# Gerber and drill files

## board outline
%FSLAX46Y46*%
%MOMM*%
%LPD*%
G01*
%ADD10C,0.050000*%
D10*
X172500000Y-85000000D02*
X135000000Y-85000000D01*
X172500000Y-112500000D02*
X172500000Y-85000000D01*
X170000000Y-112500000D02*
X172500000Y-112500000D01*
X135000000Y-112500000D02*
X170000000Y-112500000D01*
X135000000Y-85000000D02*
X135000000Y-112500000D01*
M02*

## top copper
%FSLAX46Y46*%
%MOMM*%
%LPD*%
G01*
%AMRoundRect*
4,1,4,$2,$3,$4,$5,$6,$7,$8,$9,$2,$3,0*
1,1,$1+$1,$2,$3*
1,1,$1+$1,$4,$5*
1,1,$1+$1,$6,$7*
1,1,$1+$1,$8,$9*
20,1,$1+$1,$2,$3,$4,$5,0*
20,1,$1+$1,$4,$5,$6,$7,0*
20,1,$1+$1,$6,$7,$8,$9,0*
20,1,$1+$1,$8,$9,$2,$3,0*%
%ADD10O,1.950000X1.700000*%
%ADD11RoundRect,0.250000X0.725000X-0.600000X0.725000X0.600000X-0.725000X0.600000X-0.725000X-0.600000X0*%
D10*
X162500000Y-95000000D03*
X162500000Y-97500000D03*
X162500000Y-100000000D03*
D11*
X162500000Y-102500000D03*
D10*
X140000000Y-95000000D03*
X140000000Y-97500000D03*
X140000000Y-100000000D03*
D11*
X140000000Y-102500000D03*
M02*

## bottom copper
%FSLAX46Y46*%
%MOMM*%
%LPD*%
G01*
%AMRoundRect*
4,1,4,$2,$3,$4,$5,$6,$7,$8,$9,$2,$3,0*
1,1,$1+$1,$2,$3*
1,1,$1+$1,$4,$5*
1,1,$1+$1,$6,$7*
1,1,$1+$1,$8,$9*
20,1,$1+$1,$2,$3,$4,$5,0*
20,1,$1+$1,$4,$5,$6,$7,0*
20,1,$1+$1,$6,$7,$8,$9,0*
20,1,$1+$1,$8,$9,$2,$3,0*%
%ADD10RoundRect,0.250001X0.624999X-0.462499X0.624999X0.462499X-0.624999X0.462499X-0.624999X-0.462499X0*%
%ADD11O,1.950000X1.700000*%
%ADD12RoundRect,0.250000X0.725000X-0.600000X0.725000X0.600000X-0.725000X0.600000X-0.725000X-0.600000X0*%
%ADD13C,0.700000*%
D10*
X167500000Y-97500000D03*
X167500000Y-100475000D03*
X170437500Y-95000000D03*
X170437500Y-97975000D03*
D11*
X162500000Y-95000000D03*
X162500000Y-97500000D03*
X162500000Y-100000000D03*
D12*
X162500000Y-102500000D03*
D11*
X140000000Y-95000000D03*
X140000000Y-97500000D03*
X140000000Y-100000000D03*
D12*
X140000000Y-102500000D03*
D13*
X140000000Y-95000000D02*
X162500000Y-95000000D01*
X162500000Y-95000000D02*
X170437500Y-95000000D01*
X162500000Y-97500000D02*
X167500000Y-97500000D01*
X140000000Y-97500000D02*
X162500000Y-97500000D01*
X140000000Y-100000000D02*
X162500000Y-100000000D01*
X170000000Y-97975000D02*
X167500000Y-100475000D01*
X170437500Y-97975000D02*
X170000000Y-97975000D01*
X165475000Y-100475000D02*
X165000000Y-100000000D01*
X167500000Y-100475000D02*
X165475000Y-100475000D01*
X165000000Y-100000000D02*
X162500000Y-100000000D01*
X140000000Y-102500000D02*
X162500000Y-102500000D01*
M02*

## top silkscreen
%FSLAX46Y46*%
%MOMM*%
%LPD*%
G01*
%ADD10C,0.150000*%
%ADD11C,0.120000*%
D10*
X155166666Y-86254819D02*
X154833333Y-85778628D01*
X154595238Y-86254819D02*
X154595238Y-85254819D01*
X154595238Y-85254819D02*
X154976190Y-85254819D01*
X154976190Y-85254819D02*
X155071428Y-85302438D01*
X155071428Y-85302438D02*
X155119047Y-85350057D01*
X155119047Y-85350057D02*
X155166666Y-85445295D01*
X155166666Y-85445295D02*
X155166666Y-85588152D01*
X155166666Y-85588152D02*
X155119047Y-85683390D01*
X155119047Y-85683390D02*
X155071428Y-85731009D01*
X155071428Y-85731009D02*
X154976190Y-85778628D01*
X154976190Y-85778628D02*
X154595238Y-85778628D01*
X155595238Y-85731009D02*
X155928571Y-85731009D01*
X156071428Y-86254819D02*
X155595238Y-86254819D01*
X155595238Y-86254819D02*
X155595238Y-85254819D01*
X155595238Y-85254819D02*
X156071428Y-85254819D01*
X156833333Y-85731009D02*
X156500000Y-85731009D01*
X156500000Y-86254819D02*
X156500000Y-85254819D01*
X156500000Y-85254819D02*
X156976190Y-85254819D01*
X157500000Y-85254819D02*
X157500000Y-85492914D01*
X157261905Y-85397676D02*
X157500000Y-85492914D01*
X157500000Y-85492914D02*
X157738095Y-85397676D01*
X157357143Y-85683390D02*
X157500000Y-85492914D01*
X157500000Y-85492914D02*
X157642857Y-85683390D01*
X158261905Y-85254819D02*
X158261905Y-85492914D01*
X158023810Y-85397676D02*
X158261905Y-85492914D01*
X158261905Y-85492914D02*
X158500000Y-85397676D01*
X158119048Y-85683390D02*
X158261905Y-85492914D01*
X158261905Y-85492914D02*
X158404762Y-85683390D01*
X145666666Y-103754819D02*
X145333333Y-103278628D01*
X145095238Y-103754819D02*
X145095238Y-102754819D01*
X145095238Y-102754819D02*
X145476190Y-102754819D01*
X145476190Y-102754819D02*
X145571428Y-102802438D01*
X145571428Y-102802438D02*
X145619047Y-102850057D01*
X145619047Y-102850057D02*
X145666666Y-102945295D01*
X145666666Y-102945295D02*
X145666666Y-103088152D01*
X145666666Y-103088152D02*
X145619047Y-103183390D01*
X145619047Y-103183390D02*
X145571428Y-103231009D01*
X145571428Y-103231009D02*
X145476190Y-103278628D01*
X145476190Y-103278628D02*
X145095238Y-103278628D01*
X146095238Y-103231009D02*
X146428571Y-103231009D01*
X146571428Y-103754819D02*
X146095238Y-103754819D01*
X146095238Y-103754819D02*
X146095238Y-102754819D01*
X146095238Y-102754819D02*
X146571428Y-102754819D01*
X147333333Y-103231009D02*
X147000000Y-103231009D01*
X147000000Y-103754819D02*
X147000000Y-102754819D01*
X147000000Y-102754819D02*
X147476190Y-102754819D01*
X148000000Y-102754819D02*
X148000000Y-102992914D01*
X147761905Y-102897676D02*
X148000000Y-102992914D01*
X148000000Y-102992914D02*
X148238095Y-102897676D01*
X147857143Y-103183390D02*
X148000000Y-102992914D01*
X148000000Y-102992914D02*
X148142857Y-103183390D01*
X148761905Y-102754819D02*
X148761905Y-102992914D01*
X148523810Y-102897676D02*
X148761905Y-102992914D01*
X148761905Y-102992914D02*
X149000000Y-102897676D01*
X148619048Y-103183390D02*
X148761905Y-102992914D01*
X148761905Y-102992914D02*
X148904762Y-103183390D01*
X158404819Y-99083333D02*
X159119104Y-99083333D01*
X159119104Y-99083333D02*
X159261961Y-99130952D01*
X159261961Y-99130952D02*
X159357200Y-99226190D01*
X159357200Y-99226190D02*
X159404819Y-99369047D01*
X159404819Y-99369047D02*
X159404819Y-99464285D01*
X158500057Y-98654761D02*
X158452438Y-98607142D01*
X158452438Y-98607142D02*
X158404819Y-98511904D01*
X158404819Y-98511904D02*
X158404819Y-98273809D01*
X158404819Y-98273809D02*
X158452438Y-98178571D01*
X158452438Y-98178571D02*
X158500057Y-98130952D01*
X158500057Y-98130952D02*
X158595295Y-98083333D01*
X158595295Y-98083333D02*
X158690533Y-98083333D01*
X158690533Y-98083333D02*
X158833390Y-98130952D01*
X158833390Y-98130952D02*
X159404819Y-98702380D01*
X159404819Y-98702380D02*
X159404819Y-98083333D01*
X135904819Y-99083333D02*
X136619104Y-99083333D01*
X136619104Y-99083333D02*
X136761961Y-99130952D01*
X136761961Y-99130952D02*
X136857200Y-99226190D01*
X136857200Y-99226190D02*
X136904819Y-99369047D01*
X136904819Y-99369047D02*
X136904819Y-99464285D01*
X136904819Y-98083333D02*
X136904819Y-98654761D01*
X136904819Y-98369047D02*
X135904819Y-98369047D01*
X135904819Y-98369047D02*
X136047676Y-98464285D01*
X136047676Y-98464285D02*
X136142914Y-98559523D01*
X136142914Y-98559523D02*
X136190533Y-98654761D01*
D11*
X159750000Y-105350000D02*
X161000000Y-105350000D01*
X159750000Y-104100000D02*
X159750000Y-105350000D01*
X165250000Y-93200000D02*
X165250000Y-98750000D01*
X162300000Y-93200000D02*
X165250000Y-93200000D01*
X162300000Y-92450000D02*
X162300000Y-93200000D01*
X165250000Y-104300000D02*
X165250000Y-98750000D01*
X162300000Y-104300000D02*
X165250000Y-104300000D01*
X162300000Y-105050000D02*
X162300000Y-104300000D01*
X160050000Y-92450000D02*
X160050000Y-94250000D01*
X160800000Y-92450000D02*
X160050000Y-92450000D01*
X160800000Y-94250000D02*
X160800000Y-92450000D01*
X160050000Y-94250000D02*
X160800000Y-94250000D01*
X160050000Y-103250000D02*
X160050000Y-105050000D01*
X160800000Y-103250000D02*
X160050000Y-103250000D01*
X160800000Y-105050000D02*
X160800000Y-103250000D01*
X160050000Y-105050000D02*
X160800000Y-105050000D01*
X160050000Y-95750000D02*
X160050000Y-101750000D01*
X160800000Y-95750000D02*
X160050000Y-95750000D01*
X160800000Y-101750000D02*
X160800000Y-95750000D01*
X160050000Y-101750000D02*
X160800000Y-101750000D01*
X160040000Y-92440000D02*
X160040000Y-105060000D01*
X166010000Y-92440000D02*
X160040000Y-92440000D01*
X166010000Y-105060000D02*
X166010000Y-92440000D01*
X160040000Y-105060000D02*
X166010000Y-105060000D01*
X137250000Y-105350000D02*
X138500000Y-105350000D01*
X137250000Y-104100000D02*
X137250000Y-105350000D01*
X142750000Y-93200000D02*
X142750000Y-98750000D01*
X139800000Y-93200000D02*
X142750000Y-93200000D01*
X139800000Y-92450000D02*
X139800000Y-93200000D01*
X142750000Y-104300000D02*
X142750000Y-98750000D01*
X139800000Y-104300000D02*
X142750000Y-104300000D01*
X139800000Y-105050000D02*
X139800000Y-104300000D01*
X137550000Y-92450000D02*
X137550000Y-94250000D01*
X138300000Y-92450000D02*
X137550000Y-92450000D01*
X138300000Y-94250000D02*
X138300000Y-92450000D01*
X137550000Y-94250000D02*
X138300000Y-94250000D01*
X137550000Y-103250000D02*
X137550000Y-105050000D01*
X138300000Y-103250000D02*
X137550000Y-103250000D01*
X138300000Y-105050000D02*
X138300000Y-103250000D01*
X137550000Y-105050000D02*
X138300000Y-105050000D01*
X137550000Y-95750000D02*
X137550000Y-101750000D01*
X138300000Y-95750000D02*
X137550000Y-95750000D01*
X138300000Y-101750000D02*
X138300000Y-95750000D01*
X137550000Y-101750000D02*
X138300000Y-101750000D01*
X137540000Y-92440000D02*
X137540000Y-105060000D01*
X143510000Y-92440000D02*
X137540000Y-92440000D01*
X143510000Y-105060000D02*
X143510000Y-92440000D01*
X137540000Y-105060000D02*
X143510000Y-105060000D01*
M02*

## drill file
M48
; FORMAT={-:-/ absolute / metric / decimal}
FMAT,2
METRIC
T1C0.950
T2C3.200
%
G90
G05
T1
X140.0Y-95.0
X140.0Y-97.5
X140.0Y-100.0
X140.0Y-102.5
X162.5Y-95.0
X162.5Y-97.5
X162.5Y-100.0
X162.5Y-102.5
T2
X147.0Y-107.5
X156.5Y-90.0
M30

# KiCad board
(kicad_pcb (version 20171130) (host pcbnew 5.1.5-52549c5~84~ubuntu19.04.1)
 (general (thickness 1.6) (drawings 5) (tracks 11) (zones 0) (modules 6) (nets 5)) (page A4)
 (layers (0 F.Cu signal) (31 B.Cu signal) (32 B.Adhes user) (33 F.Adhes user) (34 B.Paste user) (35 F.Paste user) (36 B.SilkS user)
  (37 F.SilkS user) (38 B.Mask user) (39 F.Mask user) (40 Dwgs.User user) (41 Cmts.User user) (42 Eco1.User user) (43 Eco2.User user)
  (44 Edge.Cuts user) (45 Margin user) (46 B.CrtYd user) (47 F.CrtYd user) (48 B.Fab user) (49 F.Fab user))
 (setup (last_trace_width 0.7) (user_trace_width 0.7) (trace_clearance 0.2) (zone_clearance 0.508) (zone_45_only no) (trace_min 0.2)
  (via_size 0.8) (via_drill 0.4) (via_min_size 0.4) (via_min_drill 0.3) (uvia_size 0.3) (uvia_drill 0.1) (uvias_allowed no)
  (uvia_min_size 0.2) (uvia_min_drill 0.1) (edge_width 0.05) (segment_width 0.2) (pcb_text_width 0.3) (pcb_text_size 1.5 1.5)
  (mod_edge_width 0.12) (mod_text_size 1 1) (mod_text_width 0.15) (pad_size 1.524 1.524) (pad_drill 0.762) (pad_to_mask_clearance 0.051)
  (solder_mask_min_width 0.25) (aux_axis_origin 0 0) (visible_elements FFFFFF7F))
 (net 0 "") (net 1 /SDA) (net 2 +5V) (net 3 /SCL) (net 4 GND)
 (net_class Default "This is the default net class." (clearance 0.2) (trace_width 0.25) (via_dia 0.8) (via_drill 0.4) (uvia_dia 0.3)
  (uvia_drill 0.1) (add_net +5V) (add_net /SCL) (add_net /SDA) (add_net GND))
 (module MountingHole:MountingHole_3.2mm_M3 (layer F.Cu) (at 156.5 90)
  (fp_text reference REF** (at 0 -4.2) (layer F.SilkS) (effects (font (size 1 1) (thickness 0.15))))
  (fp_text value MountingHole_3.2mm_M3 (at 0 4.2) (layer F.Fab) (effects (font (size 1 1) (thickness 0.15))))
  (pad 1 np_thru_hole circle (at 0 0) (size 3.2 3.2) (drill 3.2) (layers *.Cu *.Mask)))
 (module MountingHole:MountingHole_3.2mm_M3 (layer F.Cu) (at 147 107.5)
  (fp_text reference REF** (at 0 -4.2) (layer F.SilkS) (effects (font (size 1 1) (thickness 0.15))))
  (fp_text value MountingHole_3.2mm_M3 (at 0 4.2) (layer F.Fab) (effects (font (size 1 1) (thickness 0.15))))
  (pad 1 np_thru_hole circle (at 0 0) (size 3.2 3.2) (drill 3.2) (layers *.Cu *.Mask)))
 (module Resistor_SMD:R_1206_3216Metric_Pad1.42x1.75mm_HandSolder (layer B.Cu) (at 167.5 98.9875 90)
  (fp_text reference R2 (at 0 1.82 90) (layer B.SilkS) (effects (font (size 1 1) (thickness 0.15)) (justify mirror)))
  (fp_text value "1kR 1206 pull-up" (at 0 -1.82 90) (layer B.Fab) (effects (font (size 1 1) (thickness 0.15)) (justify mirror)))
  (pad 2 smd roundrect (at 1.4875 0 90) (size 1.425 1.75) (layers B.Cu B.Paste B.Mask) (roundrect_rratio 0.175439) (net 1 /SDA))
  (pad 1 smd roundrect (at -1.4875 0 90) (size 1.425 1.75) (layers B.Cu B.Paste B.Mask) (roundrect_rratio 0.175439) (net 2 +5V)))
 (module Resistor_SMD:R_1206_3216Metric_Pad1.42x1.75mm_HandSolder (layer B.Cu) (at 170.4375 96.4875 90)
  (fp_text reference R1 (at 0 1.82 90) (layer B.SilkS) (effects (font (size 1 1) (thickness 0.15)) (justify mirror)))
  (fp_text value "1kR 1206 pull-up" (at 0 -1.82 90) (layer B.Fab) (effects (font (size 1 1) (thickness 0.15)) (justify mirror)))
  (pad 2 smd roundrect (at 1.4875 0 90) (size 1.425 1.75) (layers B.Cu B.Paste B.Mask) (roundrect_rratio 0.175439) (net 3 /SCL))
  (pad 1 smd roundrect (at -1.4875 0 90) (size 1.425 1.75) (layers B.Cu B.Paste B.Mask) (roundrect_rratio 0.175439) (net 2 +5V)))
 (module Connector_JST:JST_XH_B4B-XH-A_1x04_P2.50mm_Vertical (layer F.Cu) (at 162.5 102.5 90)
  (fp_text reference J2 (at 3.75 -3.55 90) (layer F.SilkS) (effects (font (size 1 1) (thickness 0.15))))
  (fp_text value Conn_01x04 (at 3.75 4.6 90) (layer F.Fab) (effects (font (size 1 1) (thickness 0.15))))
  (fp_line (start -2.85 -2.75) (end -2.85 -1.5) (layer F.SilkS) (width 0.12))
  (fp_line (start -1.6 -2.75) (end -2.85 -2.75) (layer F.SilkS) (width 0.12))
  (fp_line (start 9.3 2.75) (end 3.75 2.75) (layer F.SilkS) (width 0.12))
  (fp_line (start 9.3 -0.2) (end 9.3 2.75) (layer F.SilkS) (width 0.12))
  (fp_line (start 10.05 -0.2) (end 9.3 -0.2) (layer F.SilkS) (width 0.12))
  (fp_line (start -1.8 2.75) (end 3.75 2.75) (layer F.SilkS) (width 0.12))
  (fp_line (start -1.8 -0.2) (end -1.8 2.75) (layer F.SilkS) (width 0.12))
  (fp_line (start -2.55 -0.2) (end -1.8 -0.2) (layer F.SilkS) (width 0.12))
  (fp_line (start 10.05 -2.45) (end 8.25 -2.45) (layer F.SilkS) (width 0.12))
  (fp_line (start 10.05 -1.7) (end 10.05 -2.45) (layer F.SilkS) (width 0.12))
  (fp_line (start 8.25 -1.7) (end 10.05 -1.7) (layer F.SilkS) (width 0.12))
  (fp_line (start 8.25 -2.45) (end 8.25 -1.7) (layer F.SilkS) (width 0.12))
  (fp_line (start -0.75 -2.45) (end -2.55 -2.45) (layer F.SilkS) (width 0.12))
  (fp_line (start -0.75 -1.7) (end -0.75 -2.45) (layer F.SilkS) (width 0.12))
  (fp_line (start -2.55 -1.7) (end -0.75 -1.7) (layer F.SilkS) (width 0.12))
  (fp_line (start -2.55 -2.45) (end -2.55 -1.7) (layer F.SilkS) (width 0.12))
  (fp_line (start 6.75 -2.45) (end 0.75 -2.45) (layer F.SilkS) (width 0.12))
  (fp_line (start 6.75 -1.7) (end 6.75 -2.45) (layer F.SilkS) (width 0.12))
  (fp_line (start 0.75 -1.7) (end 6.75 -1.7) (layer F.SilkS) (width 0.12))
  (fp_line (start 0.75 -2.45) (end 0.75 -1.7) (layer F.SilkS) (width 0.12))
  (fp_line (start 10.06 -2.46) (end -2.56 -2.46) (layer F.SilkS) (width 0.12))
  (fp_line (start 10.06 3.51) (end 10.06 -2.46) (layer F.SilkS) (width 0.12))
  (fp_line (start -2.56 3.51) (end 10.06 3.51) (layer F.SilkS) (width 0.12))
  (fp_line (start -2.56 -2.46) (end -2.56 3.51) (layer F.SilkS) (width 0.12))
  (pad 4 thru_hole oval (at 7.5 0 90) (size 1.7 1.95) (drill 0.95) (layers *.Cu *.Mask) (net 3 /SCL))
  (pad 3 thru_hole oval (at 5 0 90) (size 1.7 1.95) (drill 0.95) (layers *.Cu *.Mask) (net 1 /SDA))
  (pad 2 thru_hole oval (at 2.5 0 90) (size 1.7 1.95) (drill 0.95) (layers *.Cu *.Mask) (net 2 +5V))
  (pad 1 thru_hole roundrect (at 0 0 90) (size 1.7 1.95) (drill 0.95) (layers *.Cu *.Mask) (roundrect_rratio 0.147059) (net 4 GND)))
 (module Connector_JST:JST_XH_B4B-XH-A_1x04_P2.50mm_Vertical (layer F.Cu) (at 140 102.5 90)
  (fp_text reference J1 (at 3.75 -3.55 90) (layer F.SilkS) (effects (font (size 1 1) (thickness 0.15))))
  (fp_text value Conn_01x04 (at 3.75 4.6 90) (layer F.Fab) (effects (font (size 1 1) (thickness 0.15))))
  (fp_line (start -2.85 -2.75) (end -2.85 -1.5) (layer F.SilkS) (width 0.12))
  (fp_line (start -1.6 -2.75) (end -2.85 -2.75) (layer F.SilkS) (width 0.12))
  (fp_line (start 9.3 2.75) (end 3.75 2.75) (layer F.SilkS) (width 0.12))
  (fp_line (start 9.3 -0.2) (end 9.3 2.75) (layer F.SilkS) (width 0.12))
  (fp_line (start 10.05 -0.2) (end 9.3 -0.2) (layer F.SilkS) (width 0.12))
  (fp_line (start -1.8 2.75) (end 3.75 2.75) (layer F.SilkS) (width 0.12))
  (fp_line (start -1.8 -0.2) (end -1.8 2.75) (layer F.SilkS) (width 0.12))
  (fp_line (start -2.55 -0.2) (end -1.8 -0.2) (layer F.SilkS) (width 0.12))
  (fp_line (start 10.05 -2.45) (end 8.25 -2.45) (layer F.SilkS) (width 0.12))
  (fp_line (start 10.05 -1.7) (end 10.05 -2.45) (layer F.SilkS) (width 0.12))
  (fp_line (start 8.25 -1.7) (end 10.05 -1.7) (layer F.SilkS) (width 0.12))
  (fp_line (start 8.25 -2.45) (end 8.25 -1.7) (layer F.SilkS) (width 0.12))
  (fp_line (start -0.75 -2.45) (end -2.55 -2.45) (layer F.SilkS) (width 0.12))
  (fp_line (start -0.75 -1.7) (end -0.75 -2.45) (layer F.SilkS) (width 0.12))
  (fp_line (start -2.55 -1.7) (end -0.75 -1.7) (layer F.SilkS) (width 0.12))
  (fp_line (start -2.55 -2.45) (end -2.55 -1.7) (layer F.SilkS) (width 0.12))
  (fp_line (start 6.75 -2.45) (end 0.75 -2.45) (layer F.SilkS) (width 0.12))
  (fp_line (start 6.75 -1.7) (end 6.75 -2.45) (layer F.SilkS) (width 0.12))
  (fp_line (start 0.75 -1.7) (end 6.75 -1.7) (layer F.SilkS) (width 0.12))
  (fp_line (start 0.75 -2.45) (end 0.75 -1.7) (layer F.SilkS) (width 0.12))
  (fp_line (start 10.06 -2.46) (end -2.56 -2.46) (layer F.SilkS) (width 0.12))
  (fp_line (start 10.06 3.51) (end 10.06 -2.46) (layer F.SilkS) (width 0.12))
  (fp_line (start -2.56 3.51) (end 10.06 3.51) (layer F.SilkS) (width 0.12))
  (fp_line (start -2.56 -2.46) (end -2.56 3.51) (layer F.SilkS) (width 0.12))
  (pad 4 thru_hole oval (at 7.5 0 90) (size 1.7 1.95) (drill 0.95) (layers *.Cu *.Mask) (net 3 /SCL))
  (pad 3 thru_hole oval (at 5 0 90) (size 1.7 1.95) (drill 0.95) (layers *.Cu *.Mask) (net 1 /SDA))
  (pad 2 thru_hole oval (at 2.5 0 90) (size 1.7 1.95) (drill 0.95) (layers *.Cu *.Mask) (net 2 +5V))
  (pad 1 thru_hole roundrect (at 0 0 90) (size 1.7 1.95) (drill 0.95) (layers *.Cu *.Mask) (roundrect_rratio 0.147059) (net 4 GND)))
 (gr_line (start 172.5 85) (end 135 85) (layer Edge.Cuts) (width 0.05))
 (gr_line (start 172.5 112.5) (end 172.5 85) (layer Edge.Cuts) (width 0.05))
 (gr_line (start 170 112.5) (end 172.5 112.5) (layer Edge.Cuts) (width 0.05))
 (gr_line (start 135 112.5) (end 170 112.5) (layer Edge.Cuts) (width 0.05))
 (gr_line (start 135 85) (end 135 112.5) (layer Edge.Cuts) (width 0.05))
 (segment (start 140 95) (end 162.5 95) (width 0.7) (layer B.Cu) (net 3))
 (segment (start 162.5 95) (end 170.4375 95) (width 0.7) (layer B.Cu) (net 3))
 (segment (start 162.5 97.5) (end 167.5 97.5) (width 0.7) (layer B.Cu) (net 1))
 (segment (start 140 97.5) (end 162.5 97.5) (width 0.7) (layer B.Cu) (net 1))
 (segment (start 140 100) (end 162.5 100) (width 0.7) (layer B.Cu) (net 2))
 (segment (start 170 97.975) (end 167.5 100.475) (width 0.7) (layer B.Cu) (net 2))
 (segment (start 170.4375 97.975) (end 170 97.975) (width 0.7) (layer B.Cu) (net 2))
 (segment (start 165.475 100.475) (end 165 100) (width 0.7) (layer B.Cu) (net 2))
 (segment (start 167.5 100.475) (end 165.475 100.475) (width 0.7) (layer B.Cu) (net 2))
 (segment (start 165 100) (end 162.5 100) (width 0.7) (layer B.Cu) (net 2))
 (segment (start 140 102.5) (end 162.5 102.5) (width 0.7) (layer B.Cu) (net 4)))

